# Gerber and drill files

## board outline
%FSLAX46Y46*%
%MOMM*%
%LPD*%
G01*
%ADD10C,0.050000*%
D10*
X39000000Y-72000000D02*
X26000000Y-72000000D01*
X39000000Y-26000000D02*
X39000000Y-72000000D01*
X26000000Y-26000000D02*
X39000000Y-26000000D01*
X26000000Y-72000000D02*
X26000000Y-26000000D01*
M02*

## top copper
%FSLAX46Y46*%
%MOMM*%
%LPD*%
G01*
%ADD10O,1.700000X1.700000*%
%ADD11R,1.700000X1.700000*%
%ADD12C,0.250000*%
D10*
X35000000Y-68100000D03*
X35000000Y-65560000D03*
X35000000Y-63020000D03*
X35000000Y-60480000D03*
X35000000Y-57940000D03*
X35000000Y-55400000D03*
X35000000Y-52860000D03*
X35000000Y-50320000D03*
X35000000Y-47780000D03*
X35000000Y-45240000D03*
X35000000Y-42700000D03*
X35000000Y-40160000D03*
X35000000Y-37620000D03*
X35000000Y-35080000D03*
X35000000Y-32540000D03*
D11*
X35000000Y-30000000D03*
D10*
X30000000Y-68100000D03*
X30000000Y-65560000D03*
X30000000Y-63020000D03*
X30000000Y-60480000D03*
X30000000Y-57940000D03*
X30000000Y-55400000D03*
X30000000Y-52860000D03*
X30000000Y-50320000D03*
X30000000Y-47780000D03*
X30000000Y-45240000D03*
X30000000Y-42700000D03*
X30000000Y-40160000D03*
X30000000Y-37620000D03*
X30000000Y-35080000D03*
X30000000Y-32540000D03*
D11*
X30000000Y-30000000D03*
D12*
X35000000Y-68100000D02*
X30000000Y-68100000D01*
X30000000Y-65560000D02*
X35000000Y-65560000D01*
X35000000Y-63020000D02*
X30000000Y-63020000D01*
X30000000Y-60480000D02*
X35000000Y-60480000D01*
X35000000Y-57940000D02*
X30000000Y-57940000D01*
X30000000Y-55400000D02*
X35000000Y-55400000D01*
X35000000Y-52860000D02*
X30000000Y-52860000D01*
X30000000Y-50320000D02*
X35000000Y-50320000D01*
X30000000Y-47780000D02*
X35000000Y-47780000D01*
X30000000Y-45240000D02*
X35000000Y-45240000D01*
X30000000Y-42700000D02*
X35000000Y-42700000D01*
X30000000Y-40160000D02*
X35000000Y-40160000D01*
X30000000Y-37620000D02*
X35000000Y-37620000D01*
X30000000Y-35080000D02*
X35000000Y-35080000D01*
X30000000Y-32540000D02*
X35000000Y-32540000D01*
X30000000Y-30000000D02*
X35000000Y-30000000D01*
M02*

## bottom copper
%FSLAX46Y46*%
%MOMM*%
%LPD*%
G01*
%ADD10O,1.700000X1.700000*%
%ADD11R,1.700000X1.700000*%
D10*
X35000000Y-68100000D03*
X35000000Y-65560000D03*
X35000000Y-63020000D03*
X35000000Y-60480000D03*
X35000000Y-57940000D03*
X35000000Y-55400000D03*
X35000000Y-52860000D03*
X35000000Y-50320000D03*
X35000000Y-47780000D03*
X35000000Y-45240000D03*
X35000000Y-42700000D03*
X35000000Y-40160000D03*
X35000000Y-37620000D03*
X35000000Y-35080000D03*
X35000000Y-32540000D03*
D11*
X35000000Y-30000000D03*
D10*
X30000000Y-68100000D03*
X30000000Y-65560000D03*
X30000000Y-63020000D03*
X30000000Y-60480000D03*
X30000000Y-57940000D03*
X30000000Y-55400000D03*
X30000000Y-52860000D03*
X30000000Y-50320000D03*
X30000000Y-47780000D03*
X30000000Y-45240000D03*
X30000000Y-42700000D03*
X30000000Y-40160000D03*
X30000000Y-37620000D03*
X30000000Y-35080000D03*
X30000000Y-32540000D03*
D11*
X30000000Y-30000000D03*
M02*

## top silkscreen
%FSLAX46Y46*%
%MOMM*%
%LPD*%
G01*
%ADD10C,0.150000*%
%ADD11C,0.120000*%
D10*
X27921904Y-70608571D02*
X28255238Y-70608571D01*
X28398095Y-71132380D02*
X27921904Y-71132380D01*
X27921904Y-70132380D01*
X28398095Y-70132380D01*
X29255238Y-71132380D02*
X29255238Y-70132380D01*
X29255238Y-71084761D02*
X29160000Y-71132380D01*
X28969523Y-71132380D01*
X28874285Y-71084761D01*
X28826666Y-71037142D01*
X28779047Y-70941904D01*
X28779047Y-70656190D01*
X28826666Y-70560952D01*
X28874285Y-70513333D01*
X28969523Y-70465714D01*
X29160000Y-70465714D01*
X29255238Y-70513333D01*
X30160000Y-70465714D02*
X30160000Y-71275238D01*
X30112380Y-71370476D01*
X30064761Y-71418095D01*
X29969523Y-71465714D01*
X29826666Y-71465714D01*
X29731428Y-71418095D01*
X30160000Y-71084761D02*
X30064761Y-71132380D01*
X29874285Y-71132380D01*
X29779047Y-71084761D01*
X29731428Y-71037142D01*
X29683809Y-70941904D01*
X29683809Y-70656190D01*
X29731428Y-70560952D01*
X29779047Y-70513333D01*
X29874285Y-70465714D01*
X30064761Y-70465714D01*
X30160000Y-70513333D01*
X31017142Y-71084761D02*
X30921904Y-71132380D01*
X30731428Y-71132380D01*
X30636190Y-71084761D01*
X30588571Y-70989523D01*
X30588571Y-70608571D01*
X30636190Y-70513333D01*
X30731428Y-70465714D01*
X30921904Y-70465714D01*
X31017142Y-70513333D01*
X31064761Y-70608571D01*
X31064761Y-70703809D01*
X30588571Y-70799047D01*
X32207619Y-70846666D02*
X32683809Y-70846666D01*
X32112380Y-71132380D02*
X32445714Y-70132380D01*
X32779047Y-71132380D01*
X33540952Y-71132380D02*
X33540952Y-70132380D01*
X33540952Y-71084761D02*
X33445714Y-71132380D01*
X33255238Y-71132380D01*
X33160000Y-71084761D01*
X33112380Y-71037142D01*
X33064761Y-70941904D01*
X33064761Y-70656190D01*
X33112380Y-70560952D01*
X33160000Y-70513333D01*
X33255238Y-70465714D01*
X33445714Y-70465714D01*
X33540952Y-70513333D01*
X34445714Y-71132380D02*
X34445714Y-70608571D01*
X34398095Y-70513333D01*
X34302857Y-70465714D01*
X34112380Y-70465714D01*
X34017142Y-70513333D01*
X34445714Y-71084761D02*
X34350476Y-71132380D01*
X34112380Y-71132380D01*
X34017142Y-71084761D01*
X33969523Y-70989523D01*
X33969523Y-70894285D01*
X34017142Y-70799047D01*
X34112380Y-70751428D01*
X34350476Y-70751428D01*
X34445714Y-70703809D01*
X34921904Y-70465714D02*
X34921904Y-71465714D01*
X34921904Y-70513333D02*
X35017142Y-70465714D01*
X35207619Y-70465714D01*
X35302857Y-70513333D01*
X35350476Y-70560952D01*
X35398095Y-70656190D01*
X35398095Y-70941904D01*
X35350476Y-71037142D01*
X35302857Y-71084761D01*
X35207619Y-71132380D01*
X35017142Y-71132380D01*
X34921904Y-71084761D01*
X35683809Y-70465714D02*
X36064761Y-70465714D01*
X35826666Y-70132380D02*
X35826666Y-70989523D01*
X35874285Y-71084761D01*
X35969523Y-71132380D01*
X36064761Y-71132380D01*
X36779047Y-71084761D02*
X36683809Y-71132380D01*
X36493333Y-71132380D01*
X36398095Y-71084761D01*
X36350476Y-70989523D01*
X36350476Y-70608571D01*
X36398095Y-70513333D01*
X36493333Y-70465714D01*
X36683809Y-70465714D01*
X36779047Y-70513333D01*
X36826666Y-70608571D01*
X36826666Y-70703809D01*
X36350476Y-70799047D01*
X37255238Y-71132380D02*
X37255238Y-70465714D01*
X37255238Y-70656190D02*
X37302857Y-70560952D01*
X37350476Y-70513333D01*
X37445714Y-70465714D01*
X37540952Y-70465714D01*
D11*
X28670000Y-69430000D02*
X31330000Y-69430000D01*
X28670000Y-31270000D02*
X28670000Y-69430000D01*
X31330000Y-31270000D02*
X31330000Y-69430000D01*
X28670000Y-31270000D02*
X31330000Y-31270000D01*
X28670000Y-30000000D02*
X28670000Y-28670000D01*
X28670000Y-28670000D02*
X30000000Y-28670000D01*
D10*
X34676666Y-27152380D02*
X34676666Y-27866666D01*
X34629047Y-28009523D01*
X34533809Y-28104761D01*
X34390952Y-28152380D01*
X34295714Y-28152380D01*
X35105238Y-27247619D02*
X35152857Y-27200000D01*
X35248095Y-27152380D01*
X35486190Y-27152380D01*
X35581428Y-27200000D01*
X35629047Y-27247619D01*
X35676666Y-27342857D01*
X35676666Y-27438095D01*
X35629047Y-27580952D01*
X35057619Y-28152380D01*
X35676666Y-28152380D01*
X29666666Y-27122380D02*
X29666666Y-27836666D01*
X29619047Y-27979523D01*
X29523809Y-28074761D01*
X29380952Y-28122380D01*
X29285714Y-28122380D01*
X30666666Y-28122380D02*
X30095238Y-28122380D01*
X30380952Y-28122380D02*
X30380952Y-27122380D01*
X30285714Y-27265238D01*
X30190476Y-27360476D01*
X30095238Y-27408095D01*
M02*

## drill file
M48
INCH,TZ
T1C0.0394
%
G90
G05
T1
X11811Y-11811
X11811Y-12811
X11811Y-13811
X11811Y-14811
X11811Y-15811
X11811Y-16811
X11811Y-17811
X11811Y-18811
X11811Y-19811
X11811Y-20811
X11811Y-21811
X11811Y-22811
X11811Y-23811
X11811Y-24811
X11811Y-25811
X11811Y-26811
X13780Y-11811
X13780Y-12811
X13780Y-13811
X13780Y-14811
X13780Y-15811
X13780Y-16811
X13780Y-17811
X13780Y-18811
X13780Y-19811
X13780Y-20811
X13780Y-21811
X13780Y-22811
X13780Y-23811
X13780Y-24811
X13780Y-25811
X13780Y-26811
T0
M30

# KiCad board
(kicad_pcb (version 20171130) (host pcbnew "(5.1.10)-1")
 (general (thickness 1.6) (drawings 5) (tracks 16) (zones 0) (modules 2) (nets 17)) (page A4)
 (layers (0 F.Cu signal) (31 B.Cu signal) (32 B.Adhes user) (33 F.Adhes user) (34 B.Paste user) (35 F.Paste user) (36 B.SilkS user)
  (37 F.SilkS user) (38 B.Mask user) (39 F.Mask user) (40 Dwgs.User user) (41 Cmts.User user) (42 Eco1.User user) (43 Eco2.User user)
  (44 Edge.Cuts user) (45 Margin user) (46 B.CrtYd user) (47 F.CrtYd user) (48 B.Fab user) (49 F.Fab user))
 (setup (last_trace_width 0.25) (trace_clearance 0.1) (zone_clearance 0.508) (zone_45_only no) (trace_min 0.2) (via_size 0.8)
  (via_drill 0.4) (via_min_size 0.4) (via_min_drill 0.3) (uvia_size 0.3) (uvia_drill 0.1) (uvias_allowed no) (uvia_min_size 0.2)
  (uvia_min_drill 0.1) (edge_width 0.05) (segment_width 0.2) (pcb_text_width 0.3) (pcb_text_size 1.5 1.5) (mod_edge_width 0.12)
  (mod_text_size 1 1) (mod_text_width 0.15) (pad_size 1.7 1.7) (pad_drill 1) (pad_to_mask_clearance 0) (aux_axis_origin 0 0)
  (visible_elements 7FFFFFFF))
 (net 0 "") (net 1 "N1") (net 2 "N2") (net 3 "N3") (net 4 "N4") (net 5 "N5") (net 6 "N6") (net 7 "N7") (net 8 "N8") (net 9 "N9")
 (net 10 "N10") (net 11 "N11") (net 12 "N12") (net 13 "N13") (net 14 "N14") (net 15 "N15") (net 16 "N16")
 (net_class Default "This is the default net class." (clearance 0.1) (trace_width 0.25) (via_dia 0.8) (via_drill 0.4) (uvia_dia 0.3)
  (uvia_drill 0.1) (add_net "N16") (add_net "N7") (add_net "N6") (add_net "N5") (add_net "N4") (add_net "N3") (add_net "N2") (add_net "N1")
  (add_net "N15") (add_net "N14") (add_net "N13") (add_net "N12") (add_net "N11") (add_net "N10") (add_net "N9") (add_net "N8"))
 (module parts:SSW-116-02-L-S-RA (layer F.Cu) (at 35 30)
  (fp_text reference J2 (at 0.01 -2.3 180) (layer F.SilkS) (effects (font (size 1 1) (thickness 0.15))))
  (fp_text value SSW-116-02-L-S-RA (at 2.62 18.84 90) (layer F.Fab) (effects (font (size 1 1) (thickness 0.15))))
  (pad 16 thru_hole oval (at 0 38.1) (size 1.7 1.7) (drill 1) (layers *.Cu *.Mask) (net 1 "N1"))
  (pad 15 thru_hole oval (at 0 35.56) (size 1.7 1.7) (drill 1) (layers *.Cu *.Mask) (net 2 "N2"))
  (pad 14 thru_hole oval (at 0 33.02) (size 1.7 1.7) (drill 1) (layers *.Cu *.Mask) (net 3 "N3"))
  (pad 13 thru_hole oval (at 0 30.48) (size 1.7 1.7) (drill 1) (layers *.Cu *.Mask) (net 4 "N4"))
  (pad 12 thru_hole oval (at 0 27.94) (size 1.7 1.7) (drill 1) (layers *.Cu *.Mask) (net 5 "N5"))
  (pad 11 thru_hole oval (at 0 25.4) (size 1.7 1.7) (drill 1) (layers *.Cu *.Mask) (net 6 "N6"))
  (pad 10 thru_hole oval (at 0 22.86) (size 1.7 1.7) (drill 1) (layers *.Cu *.Mask) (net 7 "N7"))
  (pad 9 thru_hole oval (at 0 20.32) (size 1.7 1.7) (drill 1) (layers *.Cu *.Mask) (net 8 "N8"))
  (pad 8 thru_hole oval (at 0 17.78) (size 1.7 1.7) (drill 1) (layers *.Cu *.Mask) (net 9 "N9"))
  (pad 7 thru_hole oval (at 0 15.24) (size 1.7 1.7) (drill 1) (layers *.Cu *.Mask) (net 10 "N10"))
  (pad 6 thru_hole oval (at 0 12.7) (size 1.7 1.7) (drill 1) (layers *.Cu *.Mask) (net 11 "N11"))
  (pad 5 thru_hole oval (at 0 10.16) (size 1.7 1.7) (drill 1) (layers *.Cu *.Mask) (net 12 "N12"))
  (pad 4 thru_hole oval (at 0 7.62) (size 1.7 1.7) (drill 1) (layers *.Cu *.Mask) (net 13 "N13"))
  (pad 3 thru_hole oval (at 0 5.08) (size 1.7 1.7) (drill 1) (layers *.Cu *.Mask) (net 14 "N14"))
  (pad 2 thru_hole oval (at 0 2.54) (size 1.7 1.7) (drill 1) (layers *.Cu *.Mask) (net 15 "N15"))
  (pad 1 thru_hole rect (at 0 0) (size 1.7 1.7) (drill 1) (layers *.Cu *.Mask) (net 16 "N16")))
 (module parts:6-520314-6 (layer F.Cu) (at 30 30)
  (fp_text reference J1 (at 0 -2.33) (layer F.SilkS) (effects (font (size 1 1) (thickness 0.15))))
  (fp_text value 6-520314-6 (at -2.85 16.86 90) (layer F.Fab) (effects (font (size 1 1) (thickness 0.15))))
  (fp_line (start -1.33 39.43) (end 1.33 39.43) (layer F.SilkS) (width 0.12))
  (fp_line (start -1.33 1.27) (end -1.33 39.43) (layer F.SilkS) (width 0.12))
  (fp_line (start 1.33 1.27) (end 1.33 39.43) (layer F.SilkS) (width 0.12))
  (fp_line (start -1.33 1.27) (end 1.33 1.27) (layer F.SilkS) (width 0.12))
  (fp_line (start -1.33 0) (end -1.33 -1.33) (layer F.SilkS) (width 0.12))
  (fp_line (start -1.33 -1.33) (end 0 -1.33) (layer F.SilkS) (width 0.12))
  (pad 16 thru_hole oval (at 0 38.1) (size 1.7 1.7) (drill 1) (layers *.Cu *.Mask) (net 1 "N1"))
  (pad 15 thru_hole oval (at 0 35.56) (size 1.7 1.7) (drill 1) (layers *.Cu *.Mask) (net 2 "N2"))
  (pad 14 thru_hole oval (at 0 33.02) (size 1.7 1.7) (drill 1) (layers *.Cu *.Mask) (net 3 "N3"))
  (pad 13 thru_hole oval (at 0 30.48) (size 1.7 1.7) (drill 1) (layers *.Cu *.Mask) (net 4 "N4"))
  (pad 12 thru_hole oval (at 0 27.94) (size 1.7 1.7) (drill 1) (layers *.Cu *.Mask) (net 5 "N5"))
  (pad 11 thru_hole oval (at 0 25.4) (size 1.7 1.7) (drill 1) (layers *.Cu *.Mask) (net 6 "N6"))
  (pad 10 thru_hole oval (at 0 22.86) (size 1.7 1.7) (drill 1) (layers *.Cu *.Mask) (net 7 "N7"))
  (pad 9 thru_hole oval (at 0 20.32) (size 1.7 1.7) (drill 1) (layers *.Cu *.Mask) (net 8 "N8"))
  (pad 8 thru_hole oval (at 0 17.78) (size 1.7 1.7) (drill 1) (layers *.Cu *.Mask) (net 9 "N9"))
  (pad 7 thru_hole oval (at 0 15.24) (size 1.7 1.7) (drill 1) (layers *.Cu *.Mask) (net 10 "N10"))
  (pad 6 thru_hole oval (at 0 12.7) (size 1.7 1.7) (drill 1) (layers *.Cu *.Mask) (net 11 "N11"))
  (pad 5 thru_hole oval (at 0 10.16) (size 1.7 1.7) (drill 1) (layers *.Cu *.Mask) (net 12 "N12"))
  (pad 4 thru_hole oval (at 0 7.62) (size 1.7 1.7) (drill 1) (layers *.Cu *.Mask) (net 13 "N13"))
  (pad 3 thru_hole oval (at 0 5.08) (size 1.7 1.7) (drill 1) (layers *.Cu *.Mask) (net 14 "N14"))
  (pad 2 thru_hole oval (at 0 2.54) (size 1.7 1.7) (drill 1) (layers *.Cu *.Mask) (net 15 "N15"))
  (pad 1 thru_hole rect (at 0 0) (size 1.7 1.7) (drill 1) (layers *.Cu *.Mask) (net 16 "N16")))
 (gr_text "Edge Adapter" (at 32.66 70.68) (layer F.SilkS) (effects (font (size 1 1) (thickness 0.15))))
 (gr_line (start 39 72) (end 26 72) (layer Edge.Cuts) (width 0.05))
 (gr_line (start 39 26) (end 39 72) (layer Edge.Cuts) (width 0.05))
 (gr_line (start 26 26) (end 39 26) (layer Edge.Cuts) (width 0.05))
 (gr_line (start 26 72) (end 26 26) (layer Edge.Cuts) (width 0.05))
 (segment (start 35 68.1) (end 30 68.1) (width 0.25) (layer F.Cu) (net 1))
 (segment (start 30 65.56) (end 35 65.56) (width 0.25) (layer F.Cu) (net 2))
 (segment (start 35 63.02) (end 30 63.02) (width 0.25) (layer F.Cu) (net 3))
 (segment (start 30 60.48) (end 35 60.48) (width 0.25) (layer F.Cu) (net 4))
 (segment (start 35 57.94) (end 30 57.94) (width 0.25) (layer F.Cu) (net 5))
 (segment (start 30 55.4) (end 35 55.4) (width 0.25) (layer F.Cu) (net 6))
 (segment (start 35 52.86) (end 30 52.86) (width 0.25) (layer F.Cu) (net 7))
 (segment (start 30 50.32) (end 35 50.32) (width 0.25) (layer F.Cu) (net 8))
 (segment (start 30 47.78) (end 35 47.78) (width 0.25) (layer F.Cu) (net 9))
 (segment (start 30 45.24) (end 35 45.24) (width 0.25) (layer F.Cu) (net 10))
 (segment (start 30 42.7) (end 35 42.7) (width 0.25) (layer F.Cu) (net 11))
 (segment (start 30 40.16) (end 35 40.16) (width 0.25) (layer F.Cu) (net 12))
 (segment (start 30 37.62) (end 35 37.62) (width 0.25) (layer F.Cu) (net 13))
 (segment (start 30 35.08) (end 35 35.08) (width 0.25) (layer F.Cu) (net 14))
 (segment (start 30 32.54) (end 35 32.54) (width 0.25) (layer F.Cu) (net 15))
 (segment (start 30 30) (end 35 30) (width 0.25) (layer F.Cu) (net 16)))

